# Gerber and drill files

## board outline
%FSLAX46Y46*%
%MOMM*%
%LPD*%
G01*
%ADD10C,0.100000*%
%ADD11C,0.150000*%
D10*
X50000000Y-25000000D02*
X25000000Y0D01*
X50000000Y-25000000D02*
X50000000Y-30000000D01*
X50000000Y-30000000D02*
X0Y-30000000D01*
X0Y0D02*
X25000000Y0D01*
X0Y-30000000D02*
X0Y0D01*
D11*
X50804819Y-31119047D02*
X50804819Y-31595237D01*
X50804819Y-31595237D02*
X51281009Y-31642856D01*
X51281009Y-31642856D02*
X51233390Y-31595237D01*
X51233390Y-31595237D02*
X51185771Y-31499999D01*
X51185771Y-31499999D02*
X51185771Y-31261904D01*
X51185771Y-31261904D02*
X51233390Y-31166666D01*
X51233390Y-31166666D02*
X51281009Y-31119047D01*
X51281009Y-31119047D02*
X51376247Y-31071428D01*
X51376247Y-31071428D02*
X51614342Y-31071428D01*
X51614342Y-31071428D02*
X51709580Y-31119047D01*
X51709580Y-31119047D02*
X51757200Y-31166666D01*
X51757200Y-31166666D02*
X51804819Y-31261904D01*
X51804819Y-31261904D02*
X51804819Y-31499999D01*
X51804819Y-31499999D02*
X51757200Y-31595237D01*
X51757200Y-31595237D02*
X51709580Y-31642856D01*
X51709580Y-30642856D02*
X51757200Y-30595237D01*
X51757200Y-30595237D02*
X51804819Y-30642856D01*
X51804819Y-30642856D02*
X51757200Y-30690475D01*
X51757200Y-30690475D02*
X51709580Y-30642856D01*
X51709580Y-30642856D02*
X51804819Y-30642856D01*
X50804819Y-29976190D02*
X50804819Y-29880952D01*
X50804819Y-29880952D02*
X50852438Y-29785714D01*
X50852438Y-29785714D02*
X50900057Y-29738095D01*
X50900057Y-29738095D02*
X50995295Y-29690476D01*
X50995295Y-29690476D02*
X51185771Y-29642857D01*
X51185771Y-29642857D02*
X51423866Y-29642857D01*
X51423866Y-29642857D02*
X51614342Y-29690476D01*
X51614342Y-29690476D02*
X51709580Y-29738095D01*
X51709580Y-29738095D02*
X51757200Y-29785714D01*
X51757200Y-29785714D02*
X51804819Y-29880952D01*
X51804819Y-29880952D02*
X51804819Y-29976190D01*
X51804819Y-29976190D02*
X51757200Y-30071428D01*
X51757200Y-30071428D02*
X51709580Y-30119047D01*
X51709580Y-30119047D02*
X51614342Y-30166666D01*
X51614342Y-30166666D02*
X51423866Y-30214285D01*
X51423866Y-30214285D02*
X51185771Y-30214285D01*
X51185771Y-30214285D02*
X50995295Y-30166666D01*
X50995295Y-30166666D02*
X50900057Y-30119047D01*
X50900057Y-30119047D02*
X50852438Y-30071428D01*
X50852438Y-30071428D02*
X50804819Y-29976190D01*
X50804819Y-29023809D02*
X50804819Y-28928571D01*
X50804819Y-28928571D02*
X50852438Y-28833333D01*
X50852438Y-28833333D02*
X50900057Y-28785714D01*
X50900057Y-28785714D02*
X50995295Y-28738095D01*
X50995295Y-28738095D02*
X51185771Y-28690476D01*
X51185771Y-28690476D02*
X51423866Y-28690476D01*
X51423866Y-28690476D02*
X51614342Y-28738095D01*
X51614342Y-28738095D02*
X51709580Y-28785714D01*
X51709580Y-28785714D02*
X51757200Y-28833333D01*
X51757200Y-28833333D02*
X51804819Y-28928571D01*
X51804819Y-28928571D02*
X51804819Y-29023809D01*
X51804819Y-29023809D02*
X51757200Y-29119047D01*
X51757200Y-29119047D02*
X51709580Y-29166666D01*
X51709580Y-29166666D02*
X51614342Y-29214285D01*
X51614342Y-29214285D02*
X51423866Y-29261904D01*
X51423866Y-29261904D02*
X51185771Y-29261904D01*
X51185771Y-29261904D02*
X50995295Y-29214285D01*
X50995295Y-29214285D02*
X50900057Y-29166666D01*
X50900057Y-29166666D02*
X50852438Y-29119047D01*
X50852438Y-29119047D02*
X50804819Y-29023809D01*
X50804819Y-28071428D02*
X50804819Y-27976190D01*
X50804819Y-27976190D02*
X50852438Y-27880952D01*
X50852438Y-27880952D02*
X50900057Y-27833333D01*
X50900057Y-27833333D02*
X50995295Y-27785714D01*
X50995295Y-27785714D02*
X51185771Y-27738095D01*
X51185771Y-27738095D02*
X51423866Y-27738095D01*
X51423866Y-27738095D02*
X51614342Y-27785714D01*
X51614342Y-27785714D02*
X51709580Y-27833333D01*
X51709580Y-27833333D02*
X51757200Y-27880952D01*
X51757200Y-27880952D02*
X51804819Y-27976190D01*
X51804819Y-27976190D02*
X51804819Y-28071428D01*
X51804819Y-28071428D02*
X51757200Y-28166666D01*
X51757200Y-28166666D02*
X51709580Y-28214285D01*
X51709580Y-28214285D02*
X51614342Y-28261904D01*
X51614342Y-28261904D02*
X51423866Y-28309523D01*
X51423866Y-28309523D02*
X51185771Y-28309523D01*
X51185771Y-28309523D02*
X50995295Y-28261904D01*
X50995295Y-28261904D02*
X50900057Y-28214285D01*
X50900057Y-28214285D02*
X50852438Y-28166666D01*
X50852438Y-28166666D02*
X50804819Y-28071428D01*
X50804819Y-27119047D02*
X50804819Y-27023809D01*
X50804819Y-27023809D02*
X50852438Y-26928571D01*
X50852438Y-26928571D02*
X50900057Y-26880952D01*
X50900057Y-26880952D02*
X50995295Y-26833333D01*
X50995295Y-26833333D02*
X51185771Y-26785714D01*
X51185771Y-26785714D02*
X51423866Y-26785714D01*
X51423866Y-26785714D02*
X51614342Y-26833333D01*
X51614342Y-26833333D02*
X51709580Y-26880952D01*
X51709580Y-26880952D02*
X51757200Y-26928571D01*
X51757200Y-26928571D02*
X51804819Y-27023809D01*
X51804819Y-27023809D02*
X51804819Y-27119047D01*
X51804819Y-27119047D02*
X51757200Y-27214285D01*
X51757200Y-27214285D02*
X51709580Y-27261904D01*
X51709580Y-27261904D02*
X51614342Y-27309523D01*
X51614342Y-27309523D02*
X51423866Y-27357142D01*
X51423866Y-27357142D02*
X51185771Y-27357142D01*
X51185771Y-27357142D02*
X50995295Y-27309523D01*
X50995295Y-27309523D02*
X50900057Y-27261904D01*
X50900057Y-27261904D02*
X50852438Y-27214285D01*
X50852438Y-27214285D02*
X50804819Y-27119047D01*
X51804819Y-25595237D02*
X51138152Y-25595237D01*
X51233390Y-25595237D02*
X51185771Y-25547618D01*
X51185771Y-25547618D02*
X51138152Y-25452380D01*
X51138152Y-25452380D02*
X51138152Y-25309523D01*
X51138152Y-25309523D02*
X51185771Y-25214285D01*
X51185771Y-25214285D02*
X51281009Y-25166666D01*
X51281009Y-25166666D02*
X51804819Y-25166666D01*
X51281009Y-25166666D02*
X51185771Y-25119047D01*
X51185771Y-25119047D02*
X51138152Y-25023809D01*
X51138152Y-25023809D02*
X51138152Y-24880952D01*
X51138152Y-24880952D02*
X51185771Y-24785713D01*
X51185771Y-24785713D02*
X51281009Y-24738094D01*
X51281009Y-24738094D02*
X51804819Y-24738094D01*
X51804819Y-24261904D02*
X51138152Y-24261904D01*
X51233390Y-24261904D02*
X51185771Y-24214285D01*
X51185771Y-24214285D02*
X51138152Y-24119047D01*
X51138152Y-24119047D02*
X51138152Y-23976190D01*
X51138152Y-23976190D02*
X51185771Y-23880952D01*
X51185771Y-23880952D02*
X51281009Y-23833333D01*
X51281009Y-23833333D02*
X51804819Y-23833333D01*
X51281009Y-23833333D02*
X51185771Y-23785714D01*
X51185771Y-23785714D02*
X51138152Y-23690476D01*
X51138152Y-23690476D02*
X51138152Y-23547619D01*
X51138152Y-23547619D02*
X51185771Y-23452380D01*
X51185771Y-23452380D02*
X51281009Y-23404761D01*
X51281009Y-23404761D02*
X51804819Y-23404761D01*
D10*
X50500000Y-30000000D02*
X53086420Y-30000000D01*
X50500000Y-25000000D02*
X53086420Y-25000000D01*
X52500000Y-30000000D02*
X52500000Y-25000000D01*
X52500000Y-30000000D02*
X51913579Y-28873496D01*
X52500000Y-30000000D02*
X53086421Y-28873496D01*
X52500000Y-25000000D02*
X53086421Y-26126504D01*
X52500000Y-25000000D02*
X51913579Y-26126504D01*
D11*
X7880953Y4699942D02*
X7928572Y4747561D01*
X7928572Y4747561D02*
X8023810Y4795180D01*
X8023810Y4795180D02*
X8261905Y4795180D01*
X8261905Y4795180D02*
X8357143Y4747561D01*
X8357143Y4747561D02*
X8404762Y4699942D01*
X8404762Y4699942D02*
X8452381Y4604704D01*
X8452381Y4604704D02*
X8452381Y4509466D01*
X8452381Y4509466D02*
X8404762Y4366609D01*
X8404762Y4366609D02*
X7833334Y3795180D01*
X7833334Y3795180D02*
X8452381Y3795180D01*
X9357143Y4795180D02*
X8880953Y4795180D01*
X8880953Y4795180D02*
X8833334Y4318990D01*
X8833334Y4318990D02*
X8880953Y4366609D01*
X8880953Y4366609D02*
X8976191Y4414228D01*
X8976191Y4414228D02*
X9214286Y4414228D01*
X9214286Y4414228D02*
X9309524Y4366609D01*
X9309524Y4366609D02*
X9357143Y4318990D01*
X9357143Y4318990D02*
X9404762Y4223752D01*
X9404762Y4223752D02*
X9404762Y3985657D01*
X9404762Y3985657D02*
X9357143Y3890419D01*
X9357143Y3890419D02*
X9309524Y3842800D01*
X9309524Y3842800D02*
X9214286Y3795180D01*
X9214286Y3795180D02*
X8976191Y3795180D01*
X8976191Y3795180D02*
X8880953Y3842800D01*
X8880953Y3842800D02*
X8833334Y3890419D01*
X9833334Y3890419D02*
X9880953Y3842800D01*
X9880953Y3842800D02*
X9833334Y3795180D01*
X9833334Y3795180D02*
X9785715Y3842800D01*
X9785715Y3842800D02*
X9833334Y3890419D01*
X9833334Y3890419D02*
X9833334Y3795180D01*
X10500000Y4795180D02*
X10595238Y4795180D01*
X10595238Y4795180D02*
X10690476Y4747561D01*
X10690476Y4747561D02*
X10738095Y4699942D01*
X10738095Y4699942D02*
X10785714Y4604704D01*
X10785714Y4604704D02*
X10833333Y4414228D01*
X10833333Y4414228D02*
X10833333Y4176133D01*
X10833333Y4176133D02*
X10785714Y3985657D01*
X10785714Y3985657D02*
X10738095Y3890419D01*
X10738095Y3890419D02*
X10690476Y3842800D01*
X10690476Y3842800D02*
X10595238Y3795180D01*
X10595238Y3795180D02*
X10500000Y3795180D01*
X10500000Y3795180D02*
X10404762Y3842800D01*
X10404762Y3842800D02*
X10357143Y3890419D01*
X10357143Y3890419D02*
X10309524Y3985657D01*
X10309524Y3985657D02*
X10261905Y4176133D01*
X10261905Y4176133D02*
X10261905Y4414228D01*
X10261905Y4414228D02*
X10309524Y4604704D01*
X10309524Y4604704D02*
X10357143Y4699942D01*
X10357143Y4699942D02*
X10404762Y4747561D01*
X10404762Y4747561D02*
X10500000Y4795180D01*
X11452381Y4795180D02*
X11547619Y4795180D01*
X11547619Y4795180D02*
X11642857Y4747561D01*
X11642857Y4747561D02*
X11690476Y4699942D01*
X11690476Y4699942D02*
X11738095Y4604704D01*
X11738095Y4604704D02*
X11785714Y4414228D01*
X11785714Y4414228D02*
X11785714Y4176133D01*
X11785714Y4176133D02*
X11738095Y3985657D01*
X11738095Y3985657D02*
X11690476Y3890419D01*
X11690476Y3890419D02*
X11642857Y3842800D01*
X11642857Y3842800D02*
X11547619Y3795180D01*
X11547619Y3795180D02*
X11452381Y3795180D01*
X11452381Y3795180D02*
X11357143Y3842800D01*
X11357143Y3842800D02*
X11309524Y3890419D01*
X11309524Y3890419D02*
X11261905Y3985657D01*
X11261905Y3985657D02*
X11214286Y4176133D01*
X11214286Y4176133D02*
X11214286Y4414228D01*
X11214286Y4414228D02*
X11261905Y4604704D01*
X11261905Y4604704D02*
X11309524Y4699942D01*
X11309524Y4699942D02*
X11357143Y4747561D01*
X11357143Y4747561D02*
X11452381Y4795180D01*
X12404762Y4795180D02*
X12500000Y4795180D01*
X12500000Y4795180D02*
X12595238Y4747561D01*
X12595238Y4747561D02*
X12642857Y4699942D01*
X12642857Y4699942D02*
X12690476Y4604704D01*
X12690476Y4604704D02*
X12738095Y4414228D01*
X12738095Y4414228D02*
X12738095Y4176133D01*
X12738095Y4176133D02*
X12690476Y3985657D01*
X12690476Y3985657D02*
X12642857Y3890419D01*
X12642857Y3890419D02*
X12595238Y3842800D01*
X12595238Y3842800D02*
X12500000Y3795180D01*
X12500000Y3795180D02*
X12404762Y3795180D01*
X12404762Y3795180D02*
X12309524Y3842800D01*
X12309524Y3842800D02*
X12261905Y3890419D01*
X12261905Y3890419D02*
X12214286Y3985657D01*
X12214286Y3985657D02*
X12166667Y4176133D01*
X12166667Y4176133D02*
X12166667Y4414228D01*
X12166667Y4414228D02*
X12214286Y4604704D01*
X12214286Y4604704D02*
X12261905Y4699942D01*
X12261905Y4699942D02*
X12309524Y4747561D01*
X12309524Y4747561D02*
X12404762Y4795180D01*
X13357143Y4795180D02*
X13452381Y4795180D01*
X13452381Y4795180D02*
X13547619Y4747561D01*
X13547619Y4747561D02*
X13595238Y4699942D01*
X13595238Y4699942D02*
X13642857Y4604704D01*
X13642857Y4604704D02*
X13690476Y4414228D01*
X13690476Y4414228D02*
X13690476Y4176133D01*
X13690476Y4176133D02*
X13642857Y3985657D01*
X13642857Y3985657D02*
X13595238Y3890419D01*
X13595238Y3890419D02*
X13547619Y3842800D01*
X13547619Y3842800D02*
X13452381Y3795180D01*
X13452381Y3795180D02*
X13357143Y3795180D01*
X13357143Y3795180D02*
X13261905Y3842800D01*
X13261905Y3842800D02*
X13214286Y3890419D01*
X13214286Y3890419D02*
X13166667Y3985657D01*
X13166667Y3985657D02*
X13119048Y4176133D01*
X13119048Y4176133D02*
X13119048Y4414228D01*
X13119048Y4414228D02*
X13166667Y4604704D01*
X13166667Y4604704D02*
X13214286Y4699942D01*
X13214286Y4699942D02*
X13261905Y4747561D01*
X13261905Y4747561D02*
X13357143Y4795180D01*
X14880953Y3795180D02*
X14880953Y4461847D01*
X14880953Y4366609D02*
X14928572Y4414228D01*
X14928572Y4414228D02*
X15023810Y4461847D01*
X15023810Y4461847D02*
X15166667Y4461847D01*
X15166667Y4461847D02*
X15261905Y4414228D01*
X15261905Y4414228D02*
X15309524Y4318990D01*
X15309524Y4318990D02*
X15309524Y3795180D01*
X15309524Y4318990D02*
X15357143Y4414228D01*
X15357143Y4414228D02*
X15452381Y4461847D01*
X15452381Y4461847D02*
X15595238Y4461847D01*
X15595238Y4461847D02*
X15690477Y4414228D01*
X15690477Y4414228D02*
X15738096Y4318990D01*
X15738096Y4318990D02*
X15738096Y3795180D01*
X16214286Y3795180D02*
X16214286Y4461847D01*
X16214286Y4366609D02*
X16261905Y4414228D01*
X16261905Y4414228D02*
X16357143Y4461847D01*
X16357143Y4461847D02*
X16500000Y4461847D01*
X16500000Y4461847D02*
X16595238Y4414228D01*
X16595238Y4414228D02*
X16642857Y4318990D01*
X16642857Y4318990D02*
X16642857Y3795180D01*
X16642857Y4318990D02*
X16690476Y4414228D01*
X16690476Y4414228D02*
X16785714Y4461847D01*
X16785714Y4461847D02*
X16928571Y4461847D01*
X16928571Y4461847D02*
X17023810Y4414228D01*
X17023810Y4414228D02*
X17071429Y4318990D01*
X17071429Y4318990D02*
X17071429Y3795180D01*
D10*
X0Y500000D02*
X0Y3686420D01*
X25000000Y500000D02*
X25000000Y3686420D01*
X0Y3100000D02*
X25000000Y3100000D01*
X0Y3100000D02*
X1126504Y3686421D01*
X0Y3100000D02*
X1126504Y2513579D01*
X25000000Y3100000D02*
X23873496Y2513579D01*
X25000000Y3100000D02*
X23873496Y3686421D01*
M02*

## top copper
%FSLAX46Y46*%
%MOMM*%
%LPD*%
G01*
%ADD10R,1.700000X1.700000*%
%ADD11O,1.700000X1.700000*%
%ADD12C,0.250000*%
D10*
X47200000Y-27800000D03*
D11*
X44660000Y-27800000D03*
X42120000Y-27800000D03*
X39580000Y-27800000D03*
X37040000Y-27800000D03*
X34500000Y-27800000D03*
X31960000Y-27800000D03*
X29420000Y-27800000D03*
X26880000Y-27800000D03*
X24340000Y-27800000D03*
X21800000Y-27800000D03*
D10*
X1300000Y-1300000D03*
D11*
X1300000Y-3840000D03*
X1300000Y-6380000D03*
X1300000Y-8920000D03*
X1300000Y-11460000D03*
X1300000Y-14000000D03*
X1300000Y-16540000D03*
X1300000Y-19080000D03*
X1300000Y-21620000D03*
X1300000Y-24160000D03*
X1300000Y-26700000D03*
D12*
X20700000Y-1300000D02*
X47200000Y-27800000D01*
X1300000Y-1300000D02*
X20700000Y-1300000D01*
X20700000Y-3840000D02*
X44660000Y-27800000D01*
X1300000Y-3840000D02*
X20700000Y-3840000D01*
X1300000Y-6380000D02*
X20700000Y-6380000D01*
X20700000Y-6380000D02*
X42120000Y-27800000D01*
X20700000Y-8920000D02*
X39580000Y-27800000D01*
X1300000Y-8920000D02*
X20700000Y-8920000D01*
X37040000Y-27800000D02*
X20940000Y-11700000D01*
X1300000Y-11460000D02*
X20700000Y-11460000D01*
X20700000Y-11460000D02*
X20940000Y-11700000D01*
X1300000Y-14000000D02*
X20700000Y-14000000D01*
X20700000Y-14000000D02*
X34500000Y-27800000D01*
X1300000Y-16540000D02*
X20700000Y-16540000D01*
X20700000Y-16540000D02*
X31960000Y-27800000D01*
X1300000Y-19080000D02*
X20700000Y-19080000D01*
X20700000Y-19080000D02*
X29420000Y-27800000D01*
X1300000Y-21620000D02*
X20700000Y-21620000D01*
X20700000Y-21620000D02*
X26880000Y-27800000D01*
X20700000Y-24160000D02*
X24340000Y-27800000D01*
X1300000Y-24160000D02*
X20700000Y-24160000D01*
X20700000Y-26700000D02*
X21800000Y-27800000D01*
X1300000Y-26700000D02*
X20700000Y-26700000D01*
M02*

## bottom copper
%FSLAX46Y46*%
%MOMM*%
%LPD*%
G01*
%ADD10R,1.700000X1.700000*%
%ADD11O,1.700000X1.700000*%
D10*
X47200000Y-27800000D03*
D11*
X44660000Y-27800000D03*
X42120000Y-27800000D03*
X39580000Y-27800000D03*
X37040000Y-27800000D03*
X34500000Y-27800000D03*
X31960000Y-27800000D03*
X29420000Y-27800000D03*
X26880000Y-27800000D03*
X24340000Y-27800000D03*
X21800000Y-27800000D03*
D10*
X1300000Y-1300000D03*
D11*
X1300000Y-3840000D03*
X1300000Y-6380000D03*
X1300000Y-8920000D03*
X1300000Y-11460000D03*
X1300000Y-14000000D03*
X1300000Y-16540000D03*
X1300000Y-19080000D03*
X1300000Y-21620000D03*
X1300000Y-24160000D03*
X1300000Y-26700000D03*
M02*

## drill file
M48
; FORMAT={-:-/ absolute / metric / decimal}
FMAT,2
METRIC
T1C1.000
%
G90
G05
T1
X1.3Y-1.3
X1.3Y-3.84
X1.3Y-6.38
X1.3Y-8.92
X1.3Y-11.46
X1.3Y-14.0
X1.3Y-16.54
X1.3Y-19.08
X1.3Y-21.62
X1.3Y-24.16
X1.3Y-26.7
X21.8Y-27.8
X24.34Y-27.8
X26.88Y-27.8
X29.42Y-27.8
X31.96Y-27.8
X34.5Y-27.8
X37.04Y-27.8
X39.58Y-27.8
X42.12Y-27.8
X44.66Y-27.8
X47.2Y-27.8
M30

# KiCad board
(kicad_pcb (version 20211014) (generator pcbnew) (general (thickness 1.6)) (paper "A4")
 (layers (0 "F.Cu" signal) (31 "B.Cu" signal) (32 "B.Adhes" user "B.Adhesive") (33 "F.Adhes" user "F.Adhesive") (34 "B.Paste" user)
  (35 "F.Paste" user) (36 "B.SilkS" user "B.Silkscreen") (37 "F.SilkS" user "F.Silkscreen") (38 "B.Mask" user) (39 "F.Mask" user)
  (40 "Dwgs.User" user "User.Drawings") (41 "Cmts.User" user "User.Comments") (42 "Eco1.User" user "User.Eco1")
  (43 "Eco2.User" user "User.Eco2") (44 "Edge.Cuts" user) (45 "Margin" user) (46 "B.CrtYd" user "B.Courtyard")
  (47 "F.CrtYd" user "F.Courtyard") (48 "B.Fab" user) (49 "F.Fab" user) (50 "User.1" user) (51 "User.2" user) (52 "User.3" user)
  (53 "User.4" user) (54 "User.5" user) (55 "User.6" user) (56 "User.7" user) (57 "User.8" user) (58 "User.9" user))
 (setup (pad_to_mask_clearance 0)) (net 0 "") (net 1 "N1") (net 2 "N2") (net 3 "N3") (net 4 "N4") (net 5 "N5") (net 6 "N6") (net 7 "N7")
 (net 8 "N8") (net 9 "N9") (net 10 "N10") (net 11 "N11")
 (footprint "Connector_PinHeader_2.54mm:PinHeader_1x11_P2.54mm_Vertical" (layer "F.Cu") (at 47.2 27.8 -90)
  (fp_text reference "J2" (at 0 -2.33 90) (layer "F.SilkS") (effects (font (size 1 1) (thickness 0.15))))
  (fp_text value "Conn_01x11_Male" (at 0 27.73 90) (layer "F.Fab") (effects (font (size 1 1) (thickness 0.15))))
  (pad "1" thru_hole rect (at 0 0 270) (size 1.7 1.7) (drill 1) (layers *.Cu *.Mask) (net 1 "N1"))
  (pad "2" thru_hole oval (at 0 2.54 270) (size 1.7 1.7) (drill 1) (layers *.Cu *.Mask) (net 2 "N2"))
  (pad "3" thru_hole oval (at 0 5.08 270) (size 1.7 1.7) (drill 1) (layers *.Cu *.Mask) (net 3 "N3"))
  (pad "4" thru_hole oval (at 0 7.62 270) (size 1.7 1.7) (drill 1) (layers *.Cu *.Mask) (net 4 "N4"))
  (pad "5" thru_hole oval (at 0 10.16 270) (size 1.7 1.7) (drill 1) (layers *.Cu *.Mask) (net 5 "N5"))
  (pad "6" thru_hole oval (at 0 12.7 270) (size 1.7 1.7) (drill 1) (layers *.Cu *.Mask) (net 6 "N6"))
  (pad "7" thru_hole oval (at 0 15.24 270) (size 1.7 1.7) (drill 1) (layers *.Cu *.Mask) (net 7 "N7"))
  (pad "8" thru_hole oval (at 0 17.78 270) (size 1.7 1.7) (drill 1) (layers *.Cu *.Mask) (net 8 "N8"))
  (pad "9" thru_hole oval (at 0 20.32 270) (size 1.7 1.7) (drill 1) (layers *.Cu *.Mask) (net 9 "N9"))
  (pad "10" thru_hole oval (at 0 22.86 270) (size 1.7 1.7) (drill 1) (layers *.Cu *.Mask) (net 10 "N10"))
  (pad "11" thru_hole oval (at 0 25.4 270) (size 1.7 1.7) (drill 1) (layers *.Cu *.Mask) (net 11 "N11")))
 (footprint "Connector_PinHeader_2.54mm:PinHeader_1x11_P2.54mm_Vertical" (layer "F.Cu") (at 1.3 1.3)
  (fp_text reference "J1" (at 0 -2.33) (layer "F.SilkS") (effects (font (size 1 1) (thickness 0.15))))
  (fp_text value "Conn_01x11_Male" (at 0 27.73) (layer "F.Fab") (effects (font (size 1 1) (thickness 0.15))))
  (pad "1" thru_hole rect (at 0 0) (size 1.7 1.7) (drill 1) (layers *.Cu *.Mask) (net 1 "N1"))
  (pad "2" thru_hole oval (at 0 2.54) (size 1.7 1.7) (drill 1) (layers *.Cu *.Mask) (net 2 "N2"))
  (pad "3" thru_hole oval (at 0 5.08) (size 1.7 1.7) (drill 1) (layers *.Cu *.Mask) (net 3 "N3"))
  (pad "4" thru_hole oval (at 0 7.62) (size 1.7 1.7) (drill 1) (layers *.Cu *.Mask) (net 4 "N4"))
  (pad "5" thru_hole oval (at 0 10.16) (size 1.7 1.7) (drill 1) (layers *.Cu *.Mask) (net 5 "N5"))
  (pad "6" thru_hole oval (at 0 12.7) (size 1.7 1.7) (drill 1) (layers *.Cu *.Mask) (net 6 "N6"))
  (pad "7" thru_hole oval (at 0 15.24) (size 1.7 1.7) (drill 1) (layers *.Cu *.Mask) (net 7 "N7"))
  (pad "8" thru_hole oval (at 0 17.78) (size 1.7 1.7) (drill 1) (layers *.Cu *.Mask) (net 8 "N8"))
  (pad "9" thru_hole oval (at 0 20.32) (size 1.7 1.7) (drill 1) (layers *.Cu *.Mask) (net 9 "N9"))
  (pad "10" thru_hole oval (at 0 22.86) (size 1.7 1.7) (drill 1) (layers *.Cu *.Mask) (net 10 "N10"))
  (pad "11" thru_hole oval (at 0 25.4) (size 1.7 1.7) (drill 1) (layers *.Cu *.Mask) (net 11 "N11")))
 (gr_line (start 50 25) (end 25 0) (layer "Edge.Cuts") (width 0.1))
 (gr_line (start 50 25) (end 50 30) (layer "Edge.Cuts") (width 0.1))
 (gr_line (start 50 30) (end 0 30) (layer "Edge.Cuts") (width 0.1))
 (gr_line (start 0 0) (end 25 0) (layer "Edge.Cuts") (width 0.1))
 (gr_line (start 0 30) (end 0 0) (layer "Edge.Cuts") (width 0.1))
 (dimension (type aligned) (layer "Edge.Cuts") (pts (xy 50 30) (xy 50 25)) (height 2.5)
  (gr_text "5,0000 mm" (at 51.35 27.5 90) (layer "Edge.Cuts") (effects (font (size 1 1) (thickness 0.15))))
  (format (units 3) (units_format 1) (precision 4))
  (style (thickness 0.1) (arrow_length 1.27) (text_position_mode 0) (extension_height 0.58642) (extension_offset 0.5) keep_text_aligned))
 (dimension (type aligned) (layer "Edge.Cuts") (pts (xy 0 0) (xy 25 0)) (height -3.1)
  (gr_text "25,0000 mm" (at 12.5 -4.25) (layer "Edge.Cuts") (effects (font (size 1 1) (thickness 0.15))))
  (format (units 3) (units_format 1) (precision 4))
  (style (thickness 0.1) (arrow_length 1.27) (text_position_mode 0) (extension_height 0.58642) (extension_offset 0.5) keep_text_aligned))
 (segment (start 20.7 1.3) (end 47.2 27.8) (width 0.25) (layer "F.Cu") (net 1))
 (segment (start 1.3 1.3) (end 20.7 1.3) (width 0.25) (layer "F.Cu") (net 1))
 (segment (start 20.7 3.84) (end 44.66 27.8) (width 0.25) (layer "F.Cu") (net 2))
 (segment (start 1.3 3.84) (end 20.7 3.84) (width 0.25) (layer "F.Cu") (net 2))
 (segment (start 1.3 6.38) (end 20.7 6.38) (width 0.25) (layer "F.Cu") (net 3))
 (segment (start 20.7 6.38) (end 42.12 27.8) (width 0.25) (layer "F.Cu") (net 3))
 (segment (start 20.7 8.92) (end 39.58 27.8) (width 0.25) (layer "F.Cu") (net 4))
 (segment (start 1.3 8.92) (end 20.7 8.92) (width 0.25) (layer "F.Cu") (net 4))
 (segment (start 37.04 27.8) (end 20.94 11.7) (width 0.25) (layer "F.Cu") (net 5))
 (segment (start 1.3 11.46) (end 20.7 11.46) (width 0.25) (layer "F.Cu") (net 5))
 (segment (start 20.7 11.46) (end 20.94 11.7) (width 0.25) (layer "F.Cu") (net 5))
 (segment (start 1.3 14) (end 20.7 14) (width 0.25) (layer "F.Cu") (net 6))
 (segment (start 20.7 14) (end 34.5 27.8) (width 0.25) (layer "F.Cu") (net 6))
 (segment (start 1.3 16.54) (end 20.7 16.54) (width 0.25) (layer "F.Cu") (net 7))
 (segment (start 20.7 16.54) (end 31.96 27.8) (width 0.25) (layer "F.Cu") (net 7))
 (segment (start 1.3 19.08) (end 20.7 19.08) (width 0.25) (layer "F.Cu") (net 8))
 (segment (start 20.7 19.08) (end 29.42 27.8) (width 0.25) (layer "F.Cu") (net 8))
 (segment (start 1.3 21.62) (end 20.7 21.62) (width 0.25) (layer "F.Cu") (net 9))
 (segment (start 20.7 21.62) (end 26.88 27.8) (width 0.25) (layer "F.Cu") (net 9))
 (segment (start 20.7 24.16) (end 24.34 27.8) (width 0.25) (layer "F.Cu") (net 10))
 (segment (start 1.3 24.16) (end 20.7 24.16) (width 0.25) (layer "F.Cu") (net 10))
 (segment (start 20.7 26.7) (end 21.8 27.8) (width 0.25) (layer "F.Cu") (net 11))
 (segment (start 1.3 26.7) (end 20.7 26.7) (width 0.25) (layer "F.Cu") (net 11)))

